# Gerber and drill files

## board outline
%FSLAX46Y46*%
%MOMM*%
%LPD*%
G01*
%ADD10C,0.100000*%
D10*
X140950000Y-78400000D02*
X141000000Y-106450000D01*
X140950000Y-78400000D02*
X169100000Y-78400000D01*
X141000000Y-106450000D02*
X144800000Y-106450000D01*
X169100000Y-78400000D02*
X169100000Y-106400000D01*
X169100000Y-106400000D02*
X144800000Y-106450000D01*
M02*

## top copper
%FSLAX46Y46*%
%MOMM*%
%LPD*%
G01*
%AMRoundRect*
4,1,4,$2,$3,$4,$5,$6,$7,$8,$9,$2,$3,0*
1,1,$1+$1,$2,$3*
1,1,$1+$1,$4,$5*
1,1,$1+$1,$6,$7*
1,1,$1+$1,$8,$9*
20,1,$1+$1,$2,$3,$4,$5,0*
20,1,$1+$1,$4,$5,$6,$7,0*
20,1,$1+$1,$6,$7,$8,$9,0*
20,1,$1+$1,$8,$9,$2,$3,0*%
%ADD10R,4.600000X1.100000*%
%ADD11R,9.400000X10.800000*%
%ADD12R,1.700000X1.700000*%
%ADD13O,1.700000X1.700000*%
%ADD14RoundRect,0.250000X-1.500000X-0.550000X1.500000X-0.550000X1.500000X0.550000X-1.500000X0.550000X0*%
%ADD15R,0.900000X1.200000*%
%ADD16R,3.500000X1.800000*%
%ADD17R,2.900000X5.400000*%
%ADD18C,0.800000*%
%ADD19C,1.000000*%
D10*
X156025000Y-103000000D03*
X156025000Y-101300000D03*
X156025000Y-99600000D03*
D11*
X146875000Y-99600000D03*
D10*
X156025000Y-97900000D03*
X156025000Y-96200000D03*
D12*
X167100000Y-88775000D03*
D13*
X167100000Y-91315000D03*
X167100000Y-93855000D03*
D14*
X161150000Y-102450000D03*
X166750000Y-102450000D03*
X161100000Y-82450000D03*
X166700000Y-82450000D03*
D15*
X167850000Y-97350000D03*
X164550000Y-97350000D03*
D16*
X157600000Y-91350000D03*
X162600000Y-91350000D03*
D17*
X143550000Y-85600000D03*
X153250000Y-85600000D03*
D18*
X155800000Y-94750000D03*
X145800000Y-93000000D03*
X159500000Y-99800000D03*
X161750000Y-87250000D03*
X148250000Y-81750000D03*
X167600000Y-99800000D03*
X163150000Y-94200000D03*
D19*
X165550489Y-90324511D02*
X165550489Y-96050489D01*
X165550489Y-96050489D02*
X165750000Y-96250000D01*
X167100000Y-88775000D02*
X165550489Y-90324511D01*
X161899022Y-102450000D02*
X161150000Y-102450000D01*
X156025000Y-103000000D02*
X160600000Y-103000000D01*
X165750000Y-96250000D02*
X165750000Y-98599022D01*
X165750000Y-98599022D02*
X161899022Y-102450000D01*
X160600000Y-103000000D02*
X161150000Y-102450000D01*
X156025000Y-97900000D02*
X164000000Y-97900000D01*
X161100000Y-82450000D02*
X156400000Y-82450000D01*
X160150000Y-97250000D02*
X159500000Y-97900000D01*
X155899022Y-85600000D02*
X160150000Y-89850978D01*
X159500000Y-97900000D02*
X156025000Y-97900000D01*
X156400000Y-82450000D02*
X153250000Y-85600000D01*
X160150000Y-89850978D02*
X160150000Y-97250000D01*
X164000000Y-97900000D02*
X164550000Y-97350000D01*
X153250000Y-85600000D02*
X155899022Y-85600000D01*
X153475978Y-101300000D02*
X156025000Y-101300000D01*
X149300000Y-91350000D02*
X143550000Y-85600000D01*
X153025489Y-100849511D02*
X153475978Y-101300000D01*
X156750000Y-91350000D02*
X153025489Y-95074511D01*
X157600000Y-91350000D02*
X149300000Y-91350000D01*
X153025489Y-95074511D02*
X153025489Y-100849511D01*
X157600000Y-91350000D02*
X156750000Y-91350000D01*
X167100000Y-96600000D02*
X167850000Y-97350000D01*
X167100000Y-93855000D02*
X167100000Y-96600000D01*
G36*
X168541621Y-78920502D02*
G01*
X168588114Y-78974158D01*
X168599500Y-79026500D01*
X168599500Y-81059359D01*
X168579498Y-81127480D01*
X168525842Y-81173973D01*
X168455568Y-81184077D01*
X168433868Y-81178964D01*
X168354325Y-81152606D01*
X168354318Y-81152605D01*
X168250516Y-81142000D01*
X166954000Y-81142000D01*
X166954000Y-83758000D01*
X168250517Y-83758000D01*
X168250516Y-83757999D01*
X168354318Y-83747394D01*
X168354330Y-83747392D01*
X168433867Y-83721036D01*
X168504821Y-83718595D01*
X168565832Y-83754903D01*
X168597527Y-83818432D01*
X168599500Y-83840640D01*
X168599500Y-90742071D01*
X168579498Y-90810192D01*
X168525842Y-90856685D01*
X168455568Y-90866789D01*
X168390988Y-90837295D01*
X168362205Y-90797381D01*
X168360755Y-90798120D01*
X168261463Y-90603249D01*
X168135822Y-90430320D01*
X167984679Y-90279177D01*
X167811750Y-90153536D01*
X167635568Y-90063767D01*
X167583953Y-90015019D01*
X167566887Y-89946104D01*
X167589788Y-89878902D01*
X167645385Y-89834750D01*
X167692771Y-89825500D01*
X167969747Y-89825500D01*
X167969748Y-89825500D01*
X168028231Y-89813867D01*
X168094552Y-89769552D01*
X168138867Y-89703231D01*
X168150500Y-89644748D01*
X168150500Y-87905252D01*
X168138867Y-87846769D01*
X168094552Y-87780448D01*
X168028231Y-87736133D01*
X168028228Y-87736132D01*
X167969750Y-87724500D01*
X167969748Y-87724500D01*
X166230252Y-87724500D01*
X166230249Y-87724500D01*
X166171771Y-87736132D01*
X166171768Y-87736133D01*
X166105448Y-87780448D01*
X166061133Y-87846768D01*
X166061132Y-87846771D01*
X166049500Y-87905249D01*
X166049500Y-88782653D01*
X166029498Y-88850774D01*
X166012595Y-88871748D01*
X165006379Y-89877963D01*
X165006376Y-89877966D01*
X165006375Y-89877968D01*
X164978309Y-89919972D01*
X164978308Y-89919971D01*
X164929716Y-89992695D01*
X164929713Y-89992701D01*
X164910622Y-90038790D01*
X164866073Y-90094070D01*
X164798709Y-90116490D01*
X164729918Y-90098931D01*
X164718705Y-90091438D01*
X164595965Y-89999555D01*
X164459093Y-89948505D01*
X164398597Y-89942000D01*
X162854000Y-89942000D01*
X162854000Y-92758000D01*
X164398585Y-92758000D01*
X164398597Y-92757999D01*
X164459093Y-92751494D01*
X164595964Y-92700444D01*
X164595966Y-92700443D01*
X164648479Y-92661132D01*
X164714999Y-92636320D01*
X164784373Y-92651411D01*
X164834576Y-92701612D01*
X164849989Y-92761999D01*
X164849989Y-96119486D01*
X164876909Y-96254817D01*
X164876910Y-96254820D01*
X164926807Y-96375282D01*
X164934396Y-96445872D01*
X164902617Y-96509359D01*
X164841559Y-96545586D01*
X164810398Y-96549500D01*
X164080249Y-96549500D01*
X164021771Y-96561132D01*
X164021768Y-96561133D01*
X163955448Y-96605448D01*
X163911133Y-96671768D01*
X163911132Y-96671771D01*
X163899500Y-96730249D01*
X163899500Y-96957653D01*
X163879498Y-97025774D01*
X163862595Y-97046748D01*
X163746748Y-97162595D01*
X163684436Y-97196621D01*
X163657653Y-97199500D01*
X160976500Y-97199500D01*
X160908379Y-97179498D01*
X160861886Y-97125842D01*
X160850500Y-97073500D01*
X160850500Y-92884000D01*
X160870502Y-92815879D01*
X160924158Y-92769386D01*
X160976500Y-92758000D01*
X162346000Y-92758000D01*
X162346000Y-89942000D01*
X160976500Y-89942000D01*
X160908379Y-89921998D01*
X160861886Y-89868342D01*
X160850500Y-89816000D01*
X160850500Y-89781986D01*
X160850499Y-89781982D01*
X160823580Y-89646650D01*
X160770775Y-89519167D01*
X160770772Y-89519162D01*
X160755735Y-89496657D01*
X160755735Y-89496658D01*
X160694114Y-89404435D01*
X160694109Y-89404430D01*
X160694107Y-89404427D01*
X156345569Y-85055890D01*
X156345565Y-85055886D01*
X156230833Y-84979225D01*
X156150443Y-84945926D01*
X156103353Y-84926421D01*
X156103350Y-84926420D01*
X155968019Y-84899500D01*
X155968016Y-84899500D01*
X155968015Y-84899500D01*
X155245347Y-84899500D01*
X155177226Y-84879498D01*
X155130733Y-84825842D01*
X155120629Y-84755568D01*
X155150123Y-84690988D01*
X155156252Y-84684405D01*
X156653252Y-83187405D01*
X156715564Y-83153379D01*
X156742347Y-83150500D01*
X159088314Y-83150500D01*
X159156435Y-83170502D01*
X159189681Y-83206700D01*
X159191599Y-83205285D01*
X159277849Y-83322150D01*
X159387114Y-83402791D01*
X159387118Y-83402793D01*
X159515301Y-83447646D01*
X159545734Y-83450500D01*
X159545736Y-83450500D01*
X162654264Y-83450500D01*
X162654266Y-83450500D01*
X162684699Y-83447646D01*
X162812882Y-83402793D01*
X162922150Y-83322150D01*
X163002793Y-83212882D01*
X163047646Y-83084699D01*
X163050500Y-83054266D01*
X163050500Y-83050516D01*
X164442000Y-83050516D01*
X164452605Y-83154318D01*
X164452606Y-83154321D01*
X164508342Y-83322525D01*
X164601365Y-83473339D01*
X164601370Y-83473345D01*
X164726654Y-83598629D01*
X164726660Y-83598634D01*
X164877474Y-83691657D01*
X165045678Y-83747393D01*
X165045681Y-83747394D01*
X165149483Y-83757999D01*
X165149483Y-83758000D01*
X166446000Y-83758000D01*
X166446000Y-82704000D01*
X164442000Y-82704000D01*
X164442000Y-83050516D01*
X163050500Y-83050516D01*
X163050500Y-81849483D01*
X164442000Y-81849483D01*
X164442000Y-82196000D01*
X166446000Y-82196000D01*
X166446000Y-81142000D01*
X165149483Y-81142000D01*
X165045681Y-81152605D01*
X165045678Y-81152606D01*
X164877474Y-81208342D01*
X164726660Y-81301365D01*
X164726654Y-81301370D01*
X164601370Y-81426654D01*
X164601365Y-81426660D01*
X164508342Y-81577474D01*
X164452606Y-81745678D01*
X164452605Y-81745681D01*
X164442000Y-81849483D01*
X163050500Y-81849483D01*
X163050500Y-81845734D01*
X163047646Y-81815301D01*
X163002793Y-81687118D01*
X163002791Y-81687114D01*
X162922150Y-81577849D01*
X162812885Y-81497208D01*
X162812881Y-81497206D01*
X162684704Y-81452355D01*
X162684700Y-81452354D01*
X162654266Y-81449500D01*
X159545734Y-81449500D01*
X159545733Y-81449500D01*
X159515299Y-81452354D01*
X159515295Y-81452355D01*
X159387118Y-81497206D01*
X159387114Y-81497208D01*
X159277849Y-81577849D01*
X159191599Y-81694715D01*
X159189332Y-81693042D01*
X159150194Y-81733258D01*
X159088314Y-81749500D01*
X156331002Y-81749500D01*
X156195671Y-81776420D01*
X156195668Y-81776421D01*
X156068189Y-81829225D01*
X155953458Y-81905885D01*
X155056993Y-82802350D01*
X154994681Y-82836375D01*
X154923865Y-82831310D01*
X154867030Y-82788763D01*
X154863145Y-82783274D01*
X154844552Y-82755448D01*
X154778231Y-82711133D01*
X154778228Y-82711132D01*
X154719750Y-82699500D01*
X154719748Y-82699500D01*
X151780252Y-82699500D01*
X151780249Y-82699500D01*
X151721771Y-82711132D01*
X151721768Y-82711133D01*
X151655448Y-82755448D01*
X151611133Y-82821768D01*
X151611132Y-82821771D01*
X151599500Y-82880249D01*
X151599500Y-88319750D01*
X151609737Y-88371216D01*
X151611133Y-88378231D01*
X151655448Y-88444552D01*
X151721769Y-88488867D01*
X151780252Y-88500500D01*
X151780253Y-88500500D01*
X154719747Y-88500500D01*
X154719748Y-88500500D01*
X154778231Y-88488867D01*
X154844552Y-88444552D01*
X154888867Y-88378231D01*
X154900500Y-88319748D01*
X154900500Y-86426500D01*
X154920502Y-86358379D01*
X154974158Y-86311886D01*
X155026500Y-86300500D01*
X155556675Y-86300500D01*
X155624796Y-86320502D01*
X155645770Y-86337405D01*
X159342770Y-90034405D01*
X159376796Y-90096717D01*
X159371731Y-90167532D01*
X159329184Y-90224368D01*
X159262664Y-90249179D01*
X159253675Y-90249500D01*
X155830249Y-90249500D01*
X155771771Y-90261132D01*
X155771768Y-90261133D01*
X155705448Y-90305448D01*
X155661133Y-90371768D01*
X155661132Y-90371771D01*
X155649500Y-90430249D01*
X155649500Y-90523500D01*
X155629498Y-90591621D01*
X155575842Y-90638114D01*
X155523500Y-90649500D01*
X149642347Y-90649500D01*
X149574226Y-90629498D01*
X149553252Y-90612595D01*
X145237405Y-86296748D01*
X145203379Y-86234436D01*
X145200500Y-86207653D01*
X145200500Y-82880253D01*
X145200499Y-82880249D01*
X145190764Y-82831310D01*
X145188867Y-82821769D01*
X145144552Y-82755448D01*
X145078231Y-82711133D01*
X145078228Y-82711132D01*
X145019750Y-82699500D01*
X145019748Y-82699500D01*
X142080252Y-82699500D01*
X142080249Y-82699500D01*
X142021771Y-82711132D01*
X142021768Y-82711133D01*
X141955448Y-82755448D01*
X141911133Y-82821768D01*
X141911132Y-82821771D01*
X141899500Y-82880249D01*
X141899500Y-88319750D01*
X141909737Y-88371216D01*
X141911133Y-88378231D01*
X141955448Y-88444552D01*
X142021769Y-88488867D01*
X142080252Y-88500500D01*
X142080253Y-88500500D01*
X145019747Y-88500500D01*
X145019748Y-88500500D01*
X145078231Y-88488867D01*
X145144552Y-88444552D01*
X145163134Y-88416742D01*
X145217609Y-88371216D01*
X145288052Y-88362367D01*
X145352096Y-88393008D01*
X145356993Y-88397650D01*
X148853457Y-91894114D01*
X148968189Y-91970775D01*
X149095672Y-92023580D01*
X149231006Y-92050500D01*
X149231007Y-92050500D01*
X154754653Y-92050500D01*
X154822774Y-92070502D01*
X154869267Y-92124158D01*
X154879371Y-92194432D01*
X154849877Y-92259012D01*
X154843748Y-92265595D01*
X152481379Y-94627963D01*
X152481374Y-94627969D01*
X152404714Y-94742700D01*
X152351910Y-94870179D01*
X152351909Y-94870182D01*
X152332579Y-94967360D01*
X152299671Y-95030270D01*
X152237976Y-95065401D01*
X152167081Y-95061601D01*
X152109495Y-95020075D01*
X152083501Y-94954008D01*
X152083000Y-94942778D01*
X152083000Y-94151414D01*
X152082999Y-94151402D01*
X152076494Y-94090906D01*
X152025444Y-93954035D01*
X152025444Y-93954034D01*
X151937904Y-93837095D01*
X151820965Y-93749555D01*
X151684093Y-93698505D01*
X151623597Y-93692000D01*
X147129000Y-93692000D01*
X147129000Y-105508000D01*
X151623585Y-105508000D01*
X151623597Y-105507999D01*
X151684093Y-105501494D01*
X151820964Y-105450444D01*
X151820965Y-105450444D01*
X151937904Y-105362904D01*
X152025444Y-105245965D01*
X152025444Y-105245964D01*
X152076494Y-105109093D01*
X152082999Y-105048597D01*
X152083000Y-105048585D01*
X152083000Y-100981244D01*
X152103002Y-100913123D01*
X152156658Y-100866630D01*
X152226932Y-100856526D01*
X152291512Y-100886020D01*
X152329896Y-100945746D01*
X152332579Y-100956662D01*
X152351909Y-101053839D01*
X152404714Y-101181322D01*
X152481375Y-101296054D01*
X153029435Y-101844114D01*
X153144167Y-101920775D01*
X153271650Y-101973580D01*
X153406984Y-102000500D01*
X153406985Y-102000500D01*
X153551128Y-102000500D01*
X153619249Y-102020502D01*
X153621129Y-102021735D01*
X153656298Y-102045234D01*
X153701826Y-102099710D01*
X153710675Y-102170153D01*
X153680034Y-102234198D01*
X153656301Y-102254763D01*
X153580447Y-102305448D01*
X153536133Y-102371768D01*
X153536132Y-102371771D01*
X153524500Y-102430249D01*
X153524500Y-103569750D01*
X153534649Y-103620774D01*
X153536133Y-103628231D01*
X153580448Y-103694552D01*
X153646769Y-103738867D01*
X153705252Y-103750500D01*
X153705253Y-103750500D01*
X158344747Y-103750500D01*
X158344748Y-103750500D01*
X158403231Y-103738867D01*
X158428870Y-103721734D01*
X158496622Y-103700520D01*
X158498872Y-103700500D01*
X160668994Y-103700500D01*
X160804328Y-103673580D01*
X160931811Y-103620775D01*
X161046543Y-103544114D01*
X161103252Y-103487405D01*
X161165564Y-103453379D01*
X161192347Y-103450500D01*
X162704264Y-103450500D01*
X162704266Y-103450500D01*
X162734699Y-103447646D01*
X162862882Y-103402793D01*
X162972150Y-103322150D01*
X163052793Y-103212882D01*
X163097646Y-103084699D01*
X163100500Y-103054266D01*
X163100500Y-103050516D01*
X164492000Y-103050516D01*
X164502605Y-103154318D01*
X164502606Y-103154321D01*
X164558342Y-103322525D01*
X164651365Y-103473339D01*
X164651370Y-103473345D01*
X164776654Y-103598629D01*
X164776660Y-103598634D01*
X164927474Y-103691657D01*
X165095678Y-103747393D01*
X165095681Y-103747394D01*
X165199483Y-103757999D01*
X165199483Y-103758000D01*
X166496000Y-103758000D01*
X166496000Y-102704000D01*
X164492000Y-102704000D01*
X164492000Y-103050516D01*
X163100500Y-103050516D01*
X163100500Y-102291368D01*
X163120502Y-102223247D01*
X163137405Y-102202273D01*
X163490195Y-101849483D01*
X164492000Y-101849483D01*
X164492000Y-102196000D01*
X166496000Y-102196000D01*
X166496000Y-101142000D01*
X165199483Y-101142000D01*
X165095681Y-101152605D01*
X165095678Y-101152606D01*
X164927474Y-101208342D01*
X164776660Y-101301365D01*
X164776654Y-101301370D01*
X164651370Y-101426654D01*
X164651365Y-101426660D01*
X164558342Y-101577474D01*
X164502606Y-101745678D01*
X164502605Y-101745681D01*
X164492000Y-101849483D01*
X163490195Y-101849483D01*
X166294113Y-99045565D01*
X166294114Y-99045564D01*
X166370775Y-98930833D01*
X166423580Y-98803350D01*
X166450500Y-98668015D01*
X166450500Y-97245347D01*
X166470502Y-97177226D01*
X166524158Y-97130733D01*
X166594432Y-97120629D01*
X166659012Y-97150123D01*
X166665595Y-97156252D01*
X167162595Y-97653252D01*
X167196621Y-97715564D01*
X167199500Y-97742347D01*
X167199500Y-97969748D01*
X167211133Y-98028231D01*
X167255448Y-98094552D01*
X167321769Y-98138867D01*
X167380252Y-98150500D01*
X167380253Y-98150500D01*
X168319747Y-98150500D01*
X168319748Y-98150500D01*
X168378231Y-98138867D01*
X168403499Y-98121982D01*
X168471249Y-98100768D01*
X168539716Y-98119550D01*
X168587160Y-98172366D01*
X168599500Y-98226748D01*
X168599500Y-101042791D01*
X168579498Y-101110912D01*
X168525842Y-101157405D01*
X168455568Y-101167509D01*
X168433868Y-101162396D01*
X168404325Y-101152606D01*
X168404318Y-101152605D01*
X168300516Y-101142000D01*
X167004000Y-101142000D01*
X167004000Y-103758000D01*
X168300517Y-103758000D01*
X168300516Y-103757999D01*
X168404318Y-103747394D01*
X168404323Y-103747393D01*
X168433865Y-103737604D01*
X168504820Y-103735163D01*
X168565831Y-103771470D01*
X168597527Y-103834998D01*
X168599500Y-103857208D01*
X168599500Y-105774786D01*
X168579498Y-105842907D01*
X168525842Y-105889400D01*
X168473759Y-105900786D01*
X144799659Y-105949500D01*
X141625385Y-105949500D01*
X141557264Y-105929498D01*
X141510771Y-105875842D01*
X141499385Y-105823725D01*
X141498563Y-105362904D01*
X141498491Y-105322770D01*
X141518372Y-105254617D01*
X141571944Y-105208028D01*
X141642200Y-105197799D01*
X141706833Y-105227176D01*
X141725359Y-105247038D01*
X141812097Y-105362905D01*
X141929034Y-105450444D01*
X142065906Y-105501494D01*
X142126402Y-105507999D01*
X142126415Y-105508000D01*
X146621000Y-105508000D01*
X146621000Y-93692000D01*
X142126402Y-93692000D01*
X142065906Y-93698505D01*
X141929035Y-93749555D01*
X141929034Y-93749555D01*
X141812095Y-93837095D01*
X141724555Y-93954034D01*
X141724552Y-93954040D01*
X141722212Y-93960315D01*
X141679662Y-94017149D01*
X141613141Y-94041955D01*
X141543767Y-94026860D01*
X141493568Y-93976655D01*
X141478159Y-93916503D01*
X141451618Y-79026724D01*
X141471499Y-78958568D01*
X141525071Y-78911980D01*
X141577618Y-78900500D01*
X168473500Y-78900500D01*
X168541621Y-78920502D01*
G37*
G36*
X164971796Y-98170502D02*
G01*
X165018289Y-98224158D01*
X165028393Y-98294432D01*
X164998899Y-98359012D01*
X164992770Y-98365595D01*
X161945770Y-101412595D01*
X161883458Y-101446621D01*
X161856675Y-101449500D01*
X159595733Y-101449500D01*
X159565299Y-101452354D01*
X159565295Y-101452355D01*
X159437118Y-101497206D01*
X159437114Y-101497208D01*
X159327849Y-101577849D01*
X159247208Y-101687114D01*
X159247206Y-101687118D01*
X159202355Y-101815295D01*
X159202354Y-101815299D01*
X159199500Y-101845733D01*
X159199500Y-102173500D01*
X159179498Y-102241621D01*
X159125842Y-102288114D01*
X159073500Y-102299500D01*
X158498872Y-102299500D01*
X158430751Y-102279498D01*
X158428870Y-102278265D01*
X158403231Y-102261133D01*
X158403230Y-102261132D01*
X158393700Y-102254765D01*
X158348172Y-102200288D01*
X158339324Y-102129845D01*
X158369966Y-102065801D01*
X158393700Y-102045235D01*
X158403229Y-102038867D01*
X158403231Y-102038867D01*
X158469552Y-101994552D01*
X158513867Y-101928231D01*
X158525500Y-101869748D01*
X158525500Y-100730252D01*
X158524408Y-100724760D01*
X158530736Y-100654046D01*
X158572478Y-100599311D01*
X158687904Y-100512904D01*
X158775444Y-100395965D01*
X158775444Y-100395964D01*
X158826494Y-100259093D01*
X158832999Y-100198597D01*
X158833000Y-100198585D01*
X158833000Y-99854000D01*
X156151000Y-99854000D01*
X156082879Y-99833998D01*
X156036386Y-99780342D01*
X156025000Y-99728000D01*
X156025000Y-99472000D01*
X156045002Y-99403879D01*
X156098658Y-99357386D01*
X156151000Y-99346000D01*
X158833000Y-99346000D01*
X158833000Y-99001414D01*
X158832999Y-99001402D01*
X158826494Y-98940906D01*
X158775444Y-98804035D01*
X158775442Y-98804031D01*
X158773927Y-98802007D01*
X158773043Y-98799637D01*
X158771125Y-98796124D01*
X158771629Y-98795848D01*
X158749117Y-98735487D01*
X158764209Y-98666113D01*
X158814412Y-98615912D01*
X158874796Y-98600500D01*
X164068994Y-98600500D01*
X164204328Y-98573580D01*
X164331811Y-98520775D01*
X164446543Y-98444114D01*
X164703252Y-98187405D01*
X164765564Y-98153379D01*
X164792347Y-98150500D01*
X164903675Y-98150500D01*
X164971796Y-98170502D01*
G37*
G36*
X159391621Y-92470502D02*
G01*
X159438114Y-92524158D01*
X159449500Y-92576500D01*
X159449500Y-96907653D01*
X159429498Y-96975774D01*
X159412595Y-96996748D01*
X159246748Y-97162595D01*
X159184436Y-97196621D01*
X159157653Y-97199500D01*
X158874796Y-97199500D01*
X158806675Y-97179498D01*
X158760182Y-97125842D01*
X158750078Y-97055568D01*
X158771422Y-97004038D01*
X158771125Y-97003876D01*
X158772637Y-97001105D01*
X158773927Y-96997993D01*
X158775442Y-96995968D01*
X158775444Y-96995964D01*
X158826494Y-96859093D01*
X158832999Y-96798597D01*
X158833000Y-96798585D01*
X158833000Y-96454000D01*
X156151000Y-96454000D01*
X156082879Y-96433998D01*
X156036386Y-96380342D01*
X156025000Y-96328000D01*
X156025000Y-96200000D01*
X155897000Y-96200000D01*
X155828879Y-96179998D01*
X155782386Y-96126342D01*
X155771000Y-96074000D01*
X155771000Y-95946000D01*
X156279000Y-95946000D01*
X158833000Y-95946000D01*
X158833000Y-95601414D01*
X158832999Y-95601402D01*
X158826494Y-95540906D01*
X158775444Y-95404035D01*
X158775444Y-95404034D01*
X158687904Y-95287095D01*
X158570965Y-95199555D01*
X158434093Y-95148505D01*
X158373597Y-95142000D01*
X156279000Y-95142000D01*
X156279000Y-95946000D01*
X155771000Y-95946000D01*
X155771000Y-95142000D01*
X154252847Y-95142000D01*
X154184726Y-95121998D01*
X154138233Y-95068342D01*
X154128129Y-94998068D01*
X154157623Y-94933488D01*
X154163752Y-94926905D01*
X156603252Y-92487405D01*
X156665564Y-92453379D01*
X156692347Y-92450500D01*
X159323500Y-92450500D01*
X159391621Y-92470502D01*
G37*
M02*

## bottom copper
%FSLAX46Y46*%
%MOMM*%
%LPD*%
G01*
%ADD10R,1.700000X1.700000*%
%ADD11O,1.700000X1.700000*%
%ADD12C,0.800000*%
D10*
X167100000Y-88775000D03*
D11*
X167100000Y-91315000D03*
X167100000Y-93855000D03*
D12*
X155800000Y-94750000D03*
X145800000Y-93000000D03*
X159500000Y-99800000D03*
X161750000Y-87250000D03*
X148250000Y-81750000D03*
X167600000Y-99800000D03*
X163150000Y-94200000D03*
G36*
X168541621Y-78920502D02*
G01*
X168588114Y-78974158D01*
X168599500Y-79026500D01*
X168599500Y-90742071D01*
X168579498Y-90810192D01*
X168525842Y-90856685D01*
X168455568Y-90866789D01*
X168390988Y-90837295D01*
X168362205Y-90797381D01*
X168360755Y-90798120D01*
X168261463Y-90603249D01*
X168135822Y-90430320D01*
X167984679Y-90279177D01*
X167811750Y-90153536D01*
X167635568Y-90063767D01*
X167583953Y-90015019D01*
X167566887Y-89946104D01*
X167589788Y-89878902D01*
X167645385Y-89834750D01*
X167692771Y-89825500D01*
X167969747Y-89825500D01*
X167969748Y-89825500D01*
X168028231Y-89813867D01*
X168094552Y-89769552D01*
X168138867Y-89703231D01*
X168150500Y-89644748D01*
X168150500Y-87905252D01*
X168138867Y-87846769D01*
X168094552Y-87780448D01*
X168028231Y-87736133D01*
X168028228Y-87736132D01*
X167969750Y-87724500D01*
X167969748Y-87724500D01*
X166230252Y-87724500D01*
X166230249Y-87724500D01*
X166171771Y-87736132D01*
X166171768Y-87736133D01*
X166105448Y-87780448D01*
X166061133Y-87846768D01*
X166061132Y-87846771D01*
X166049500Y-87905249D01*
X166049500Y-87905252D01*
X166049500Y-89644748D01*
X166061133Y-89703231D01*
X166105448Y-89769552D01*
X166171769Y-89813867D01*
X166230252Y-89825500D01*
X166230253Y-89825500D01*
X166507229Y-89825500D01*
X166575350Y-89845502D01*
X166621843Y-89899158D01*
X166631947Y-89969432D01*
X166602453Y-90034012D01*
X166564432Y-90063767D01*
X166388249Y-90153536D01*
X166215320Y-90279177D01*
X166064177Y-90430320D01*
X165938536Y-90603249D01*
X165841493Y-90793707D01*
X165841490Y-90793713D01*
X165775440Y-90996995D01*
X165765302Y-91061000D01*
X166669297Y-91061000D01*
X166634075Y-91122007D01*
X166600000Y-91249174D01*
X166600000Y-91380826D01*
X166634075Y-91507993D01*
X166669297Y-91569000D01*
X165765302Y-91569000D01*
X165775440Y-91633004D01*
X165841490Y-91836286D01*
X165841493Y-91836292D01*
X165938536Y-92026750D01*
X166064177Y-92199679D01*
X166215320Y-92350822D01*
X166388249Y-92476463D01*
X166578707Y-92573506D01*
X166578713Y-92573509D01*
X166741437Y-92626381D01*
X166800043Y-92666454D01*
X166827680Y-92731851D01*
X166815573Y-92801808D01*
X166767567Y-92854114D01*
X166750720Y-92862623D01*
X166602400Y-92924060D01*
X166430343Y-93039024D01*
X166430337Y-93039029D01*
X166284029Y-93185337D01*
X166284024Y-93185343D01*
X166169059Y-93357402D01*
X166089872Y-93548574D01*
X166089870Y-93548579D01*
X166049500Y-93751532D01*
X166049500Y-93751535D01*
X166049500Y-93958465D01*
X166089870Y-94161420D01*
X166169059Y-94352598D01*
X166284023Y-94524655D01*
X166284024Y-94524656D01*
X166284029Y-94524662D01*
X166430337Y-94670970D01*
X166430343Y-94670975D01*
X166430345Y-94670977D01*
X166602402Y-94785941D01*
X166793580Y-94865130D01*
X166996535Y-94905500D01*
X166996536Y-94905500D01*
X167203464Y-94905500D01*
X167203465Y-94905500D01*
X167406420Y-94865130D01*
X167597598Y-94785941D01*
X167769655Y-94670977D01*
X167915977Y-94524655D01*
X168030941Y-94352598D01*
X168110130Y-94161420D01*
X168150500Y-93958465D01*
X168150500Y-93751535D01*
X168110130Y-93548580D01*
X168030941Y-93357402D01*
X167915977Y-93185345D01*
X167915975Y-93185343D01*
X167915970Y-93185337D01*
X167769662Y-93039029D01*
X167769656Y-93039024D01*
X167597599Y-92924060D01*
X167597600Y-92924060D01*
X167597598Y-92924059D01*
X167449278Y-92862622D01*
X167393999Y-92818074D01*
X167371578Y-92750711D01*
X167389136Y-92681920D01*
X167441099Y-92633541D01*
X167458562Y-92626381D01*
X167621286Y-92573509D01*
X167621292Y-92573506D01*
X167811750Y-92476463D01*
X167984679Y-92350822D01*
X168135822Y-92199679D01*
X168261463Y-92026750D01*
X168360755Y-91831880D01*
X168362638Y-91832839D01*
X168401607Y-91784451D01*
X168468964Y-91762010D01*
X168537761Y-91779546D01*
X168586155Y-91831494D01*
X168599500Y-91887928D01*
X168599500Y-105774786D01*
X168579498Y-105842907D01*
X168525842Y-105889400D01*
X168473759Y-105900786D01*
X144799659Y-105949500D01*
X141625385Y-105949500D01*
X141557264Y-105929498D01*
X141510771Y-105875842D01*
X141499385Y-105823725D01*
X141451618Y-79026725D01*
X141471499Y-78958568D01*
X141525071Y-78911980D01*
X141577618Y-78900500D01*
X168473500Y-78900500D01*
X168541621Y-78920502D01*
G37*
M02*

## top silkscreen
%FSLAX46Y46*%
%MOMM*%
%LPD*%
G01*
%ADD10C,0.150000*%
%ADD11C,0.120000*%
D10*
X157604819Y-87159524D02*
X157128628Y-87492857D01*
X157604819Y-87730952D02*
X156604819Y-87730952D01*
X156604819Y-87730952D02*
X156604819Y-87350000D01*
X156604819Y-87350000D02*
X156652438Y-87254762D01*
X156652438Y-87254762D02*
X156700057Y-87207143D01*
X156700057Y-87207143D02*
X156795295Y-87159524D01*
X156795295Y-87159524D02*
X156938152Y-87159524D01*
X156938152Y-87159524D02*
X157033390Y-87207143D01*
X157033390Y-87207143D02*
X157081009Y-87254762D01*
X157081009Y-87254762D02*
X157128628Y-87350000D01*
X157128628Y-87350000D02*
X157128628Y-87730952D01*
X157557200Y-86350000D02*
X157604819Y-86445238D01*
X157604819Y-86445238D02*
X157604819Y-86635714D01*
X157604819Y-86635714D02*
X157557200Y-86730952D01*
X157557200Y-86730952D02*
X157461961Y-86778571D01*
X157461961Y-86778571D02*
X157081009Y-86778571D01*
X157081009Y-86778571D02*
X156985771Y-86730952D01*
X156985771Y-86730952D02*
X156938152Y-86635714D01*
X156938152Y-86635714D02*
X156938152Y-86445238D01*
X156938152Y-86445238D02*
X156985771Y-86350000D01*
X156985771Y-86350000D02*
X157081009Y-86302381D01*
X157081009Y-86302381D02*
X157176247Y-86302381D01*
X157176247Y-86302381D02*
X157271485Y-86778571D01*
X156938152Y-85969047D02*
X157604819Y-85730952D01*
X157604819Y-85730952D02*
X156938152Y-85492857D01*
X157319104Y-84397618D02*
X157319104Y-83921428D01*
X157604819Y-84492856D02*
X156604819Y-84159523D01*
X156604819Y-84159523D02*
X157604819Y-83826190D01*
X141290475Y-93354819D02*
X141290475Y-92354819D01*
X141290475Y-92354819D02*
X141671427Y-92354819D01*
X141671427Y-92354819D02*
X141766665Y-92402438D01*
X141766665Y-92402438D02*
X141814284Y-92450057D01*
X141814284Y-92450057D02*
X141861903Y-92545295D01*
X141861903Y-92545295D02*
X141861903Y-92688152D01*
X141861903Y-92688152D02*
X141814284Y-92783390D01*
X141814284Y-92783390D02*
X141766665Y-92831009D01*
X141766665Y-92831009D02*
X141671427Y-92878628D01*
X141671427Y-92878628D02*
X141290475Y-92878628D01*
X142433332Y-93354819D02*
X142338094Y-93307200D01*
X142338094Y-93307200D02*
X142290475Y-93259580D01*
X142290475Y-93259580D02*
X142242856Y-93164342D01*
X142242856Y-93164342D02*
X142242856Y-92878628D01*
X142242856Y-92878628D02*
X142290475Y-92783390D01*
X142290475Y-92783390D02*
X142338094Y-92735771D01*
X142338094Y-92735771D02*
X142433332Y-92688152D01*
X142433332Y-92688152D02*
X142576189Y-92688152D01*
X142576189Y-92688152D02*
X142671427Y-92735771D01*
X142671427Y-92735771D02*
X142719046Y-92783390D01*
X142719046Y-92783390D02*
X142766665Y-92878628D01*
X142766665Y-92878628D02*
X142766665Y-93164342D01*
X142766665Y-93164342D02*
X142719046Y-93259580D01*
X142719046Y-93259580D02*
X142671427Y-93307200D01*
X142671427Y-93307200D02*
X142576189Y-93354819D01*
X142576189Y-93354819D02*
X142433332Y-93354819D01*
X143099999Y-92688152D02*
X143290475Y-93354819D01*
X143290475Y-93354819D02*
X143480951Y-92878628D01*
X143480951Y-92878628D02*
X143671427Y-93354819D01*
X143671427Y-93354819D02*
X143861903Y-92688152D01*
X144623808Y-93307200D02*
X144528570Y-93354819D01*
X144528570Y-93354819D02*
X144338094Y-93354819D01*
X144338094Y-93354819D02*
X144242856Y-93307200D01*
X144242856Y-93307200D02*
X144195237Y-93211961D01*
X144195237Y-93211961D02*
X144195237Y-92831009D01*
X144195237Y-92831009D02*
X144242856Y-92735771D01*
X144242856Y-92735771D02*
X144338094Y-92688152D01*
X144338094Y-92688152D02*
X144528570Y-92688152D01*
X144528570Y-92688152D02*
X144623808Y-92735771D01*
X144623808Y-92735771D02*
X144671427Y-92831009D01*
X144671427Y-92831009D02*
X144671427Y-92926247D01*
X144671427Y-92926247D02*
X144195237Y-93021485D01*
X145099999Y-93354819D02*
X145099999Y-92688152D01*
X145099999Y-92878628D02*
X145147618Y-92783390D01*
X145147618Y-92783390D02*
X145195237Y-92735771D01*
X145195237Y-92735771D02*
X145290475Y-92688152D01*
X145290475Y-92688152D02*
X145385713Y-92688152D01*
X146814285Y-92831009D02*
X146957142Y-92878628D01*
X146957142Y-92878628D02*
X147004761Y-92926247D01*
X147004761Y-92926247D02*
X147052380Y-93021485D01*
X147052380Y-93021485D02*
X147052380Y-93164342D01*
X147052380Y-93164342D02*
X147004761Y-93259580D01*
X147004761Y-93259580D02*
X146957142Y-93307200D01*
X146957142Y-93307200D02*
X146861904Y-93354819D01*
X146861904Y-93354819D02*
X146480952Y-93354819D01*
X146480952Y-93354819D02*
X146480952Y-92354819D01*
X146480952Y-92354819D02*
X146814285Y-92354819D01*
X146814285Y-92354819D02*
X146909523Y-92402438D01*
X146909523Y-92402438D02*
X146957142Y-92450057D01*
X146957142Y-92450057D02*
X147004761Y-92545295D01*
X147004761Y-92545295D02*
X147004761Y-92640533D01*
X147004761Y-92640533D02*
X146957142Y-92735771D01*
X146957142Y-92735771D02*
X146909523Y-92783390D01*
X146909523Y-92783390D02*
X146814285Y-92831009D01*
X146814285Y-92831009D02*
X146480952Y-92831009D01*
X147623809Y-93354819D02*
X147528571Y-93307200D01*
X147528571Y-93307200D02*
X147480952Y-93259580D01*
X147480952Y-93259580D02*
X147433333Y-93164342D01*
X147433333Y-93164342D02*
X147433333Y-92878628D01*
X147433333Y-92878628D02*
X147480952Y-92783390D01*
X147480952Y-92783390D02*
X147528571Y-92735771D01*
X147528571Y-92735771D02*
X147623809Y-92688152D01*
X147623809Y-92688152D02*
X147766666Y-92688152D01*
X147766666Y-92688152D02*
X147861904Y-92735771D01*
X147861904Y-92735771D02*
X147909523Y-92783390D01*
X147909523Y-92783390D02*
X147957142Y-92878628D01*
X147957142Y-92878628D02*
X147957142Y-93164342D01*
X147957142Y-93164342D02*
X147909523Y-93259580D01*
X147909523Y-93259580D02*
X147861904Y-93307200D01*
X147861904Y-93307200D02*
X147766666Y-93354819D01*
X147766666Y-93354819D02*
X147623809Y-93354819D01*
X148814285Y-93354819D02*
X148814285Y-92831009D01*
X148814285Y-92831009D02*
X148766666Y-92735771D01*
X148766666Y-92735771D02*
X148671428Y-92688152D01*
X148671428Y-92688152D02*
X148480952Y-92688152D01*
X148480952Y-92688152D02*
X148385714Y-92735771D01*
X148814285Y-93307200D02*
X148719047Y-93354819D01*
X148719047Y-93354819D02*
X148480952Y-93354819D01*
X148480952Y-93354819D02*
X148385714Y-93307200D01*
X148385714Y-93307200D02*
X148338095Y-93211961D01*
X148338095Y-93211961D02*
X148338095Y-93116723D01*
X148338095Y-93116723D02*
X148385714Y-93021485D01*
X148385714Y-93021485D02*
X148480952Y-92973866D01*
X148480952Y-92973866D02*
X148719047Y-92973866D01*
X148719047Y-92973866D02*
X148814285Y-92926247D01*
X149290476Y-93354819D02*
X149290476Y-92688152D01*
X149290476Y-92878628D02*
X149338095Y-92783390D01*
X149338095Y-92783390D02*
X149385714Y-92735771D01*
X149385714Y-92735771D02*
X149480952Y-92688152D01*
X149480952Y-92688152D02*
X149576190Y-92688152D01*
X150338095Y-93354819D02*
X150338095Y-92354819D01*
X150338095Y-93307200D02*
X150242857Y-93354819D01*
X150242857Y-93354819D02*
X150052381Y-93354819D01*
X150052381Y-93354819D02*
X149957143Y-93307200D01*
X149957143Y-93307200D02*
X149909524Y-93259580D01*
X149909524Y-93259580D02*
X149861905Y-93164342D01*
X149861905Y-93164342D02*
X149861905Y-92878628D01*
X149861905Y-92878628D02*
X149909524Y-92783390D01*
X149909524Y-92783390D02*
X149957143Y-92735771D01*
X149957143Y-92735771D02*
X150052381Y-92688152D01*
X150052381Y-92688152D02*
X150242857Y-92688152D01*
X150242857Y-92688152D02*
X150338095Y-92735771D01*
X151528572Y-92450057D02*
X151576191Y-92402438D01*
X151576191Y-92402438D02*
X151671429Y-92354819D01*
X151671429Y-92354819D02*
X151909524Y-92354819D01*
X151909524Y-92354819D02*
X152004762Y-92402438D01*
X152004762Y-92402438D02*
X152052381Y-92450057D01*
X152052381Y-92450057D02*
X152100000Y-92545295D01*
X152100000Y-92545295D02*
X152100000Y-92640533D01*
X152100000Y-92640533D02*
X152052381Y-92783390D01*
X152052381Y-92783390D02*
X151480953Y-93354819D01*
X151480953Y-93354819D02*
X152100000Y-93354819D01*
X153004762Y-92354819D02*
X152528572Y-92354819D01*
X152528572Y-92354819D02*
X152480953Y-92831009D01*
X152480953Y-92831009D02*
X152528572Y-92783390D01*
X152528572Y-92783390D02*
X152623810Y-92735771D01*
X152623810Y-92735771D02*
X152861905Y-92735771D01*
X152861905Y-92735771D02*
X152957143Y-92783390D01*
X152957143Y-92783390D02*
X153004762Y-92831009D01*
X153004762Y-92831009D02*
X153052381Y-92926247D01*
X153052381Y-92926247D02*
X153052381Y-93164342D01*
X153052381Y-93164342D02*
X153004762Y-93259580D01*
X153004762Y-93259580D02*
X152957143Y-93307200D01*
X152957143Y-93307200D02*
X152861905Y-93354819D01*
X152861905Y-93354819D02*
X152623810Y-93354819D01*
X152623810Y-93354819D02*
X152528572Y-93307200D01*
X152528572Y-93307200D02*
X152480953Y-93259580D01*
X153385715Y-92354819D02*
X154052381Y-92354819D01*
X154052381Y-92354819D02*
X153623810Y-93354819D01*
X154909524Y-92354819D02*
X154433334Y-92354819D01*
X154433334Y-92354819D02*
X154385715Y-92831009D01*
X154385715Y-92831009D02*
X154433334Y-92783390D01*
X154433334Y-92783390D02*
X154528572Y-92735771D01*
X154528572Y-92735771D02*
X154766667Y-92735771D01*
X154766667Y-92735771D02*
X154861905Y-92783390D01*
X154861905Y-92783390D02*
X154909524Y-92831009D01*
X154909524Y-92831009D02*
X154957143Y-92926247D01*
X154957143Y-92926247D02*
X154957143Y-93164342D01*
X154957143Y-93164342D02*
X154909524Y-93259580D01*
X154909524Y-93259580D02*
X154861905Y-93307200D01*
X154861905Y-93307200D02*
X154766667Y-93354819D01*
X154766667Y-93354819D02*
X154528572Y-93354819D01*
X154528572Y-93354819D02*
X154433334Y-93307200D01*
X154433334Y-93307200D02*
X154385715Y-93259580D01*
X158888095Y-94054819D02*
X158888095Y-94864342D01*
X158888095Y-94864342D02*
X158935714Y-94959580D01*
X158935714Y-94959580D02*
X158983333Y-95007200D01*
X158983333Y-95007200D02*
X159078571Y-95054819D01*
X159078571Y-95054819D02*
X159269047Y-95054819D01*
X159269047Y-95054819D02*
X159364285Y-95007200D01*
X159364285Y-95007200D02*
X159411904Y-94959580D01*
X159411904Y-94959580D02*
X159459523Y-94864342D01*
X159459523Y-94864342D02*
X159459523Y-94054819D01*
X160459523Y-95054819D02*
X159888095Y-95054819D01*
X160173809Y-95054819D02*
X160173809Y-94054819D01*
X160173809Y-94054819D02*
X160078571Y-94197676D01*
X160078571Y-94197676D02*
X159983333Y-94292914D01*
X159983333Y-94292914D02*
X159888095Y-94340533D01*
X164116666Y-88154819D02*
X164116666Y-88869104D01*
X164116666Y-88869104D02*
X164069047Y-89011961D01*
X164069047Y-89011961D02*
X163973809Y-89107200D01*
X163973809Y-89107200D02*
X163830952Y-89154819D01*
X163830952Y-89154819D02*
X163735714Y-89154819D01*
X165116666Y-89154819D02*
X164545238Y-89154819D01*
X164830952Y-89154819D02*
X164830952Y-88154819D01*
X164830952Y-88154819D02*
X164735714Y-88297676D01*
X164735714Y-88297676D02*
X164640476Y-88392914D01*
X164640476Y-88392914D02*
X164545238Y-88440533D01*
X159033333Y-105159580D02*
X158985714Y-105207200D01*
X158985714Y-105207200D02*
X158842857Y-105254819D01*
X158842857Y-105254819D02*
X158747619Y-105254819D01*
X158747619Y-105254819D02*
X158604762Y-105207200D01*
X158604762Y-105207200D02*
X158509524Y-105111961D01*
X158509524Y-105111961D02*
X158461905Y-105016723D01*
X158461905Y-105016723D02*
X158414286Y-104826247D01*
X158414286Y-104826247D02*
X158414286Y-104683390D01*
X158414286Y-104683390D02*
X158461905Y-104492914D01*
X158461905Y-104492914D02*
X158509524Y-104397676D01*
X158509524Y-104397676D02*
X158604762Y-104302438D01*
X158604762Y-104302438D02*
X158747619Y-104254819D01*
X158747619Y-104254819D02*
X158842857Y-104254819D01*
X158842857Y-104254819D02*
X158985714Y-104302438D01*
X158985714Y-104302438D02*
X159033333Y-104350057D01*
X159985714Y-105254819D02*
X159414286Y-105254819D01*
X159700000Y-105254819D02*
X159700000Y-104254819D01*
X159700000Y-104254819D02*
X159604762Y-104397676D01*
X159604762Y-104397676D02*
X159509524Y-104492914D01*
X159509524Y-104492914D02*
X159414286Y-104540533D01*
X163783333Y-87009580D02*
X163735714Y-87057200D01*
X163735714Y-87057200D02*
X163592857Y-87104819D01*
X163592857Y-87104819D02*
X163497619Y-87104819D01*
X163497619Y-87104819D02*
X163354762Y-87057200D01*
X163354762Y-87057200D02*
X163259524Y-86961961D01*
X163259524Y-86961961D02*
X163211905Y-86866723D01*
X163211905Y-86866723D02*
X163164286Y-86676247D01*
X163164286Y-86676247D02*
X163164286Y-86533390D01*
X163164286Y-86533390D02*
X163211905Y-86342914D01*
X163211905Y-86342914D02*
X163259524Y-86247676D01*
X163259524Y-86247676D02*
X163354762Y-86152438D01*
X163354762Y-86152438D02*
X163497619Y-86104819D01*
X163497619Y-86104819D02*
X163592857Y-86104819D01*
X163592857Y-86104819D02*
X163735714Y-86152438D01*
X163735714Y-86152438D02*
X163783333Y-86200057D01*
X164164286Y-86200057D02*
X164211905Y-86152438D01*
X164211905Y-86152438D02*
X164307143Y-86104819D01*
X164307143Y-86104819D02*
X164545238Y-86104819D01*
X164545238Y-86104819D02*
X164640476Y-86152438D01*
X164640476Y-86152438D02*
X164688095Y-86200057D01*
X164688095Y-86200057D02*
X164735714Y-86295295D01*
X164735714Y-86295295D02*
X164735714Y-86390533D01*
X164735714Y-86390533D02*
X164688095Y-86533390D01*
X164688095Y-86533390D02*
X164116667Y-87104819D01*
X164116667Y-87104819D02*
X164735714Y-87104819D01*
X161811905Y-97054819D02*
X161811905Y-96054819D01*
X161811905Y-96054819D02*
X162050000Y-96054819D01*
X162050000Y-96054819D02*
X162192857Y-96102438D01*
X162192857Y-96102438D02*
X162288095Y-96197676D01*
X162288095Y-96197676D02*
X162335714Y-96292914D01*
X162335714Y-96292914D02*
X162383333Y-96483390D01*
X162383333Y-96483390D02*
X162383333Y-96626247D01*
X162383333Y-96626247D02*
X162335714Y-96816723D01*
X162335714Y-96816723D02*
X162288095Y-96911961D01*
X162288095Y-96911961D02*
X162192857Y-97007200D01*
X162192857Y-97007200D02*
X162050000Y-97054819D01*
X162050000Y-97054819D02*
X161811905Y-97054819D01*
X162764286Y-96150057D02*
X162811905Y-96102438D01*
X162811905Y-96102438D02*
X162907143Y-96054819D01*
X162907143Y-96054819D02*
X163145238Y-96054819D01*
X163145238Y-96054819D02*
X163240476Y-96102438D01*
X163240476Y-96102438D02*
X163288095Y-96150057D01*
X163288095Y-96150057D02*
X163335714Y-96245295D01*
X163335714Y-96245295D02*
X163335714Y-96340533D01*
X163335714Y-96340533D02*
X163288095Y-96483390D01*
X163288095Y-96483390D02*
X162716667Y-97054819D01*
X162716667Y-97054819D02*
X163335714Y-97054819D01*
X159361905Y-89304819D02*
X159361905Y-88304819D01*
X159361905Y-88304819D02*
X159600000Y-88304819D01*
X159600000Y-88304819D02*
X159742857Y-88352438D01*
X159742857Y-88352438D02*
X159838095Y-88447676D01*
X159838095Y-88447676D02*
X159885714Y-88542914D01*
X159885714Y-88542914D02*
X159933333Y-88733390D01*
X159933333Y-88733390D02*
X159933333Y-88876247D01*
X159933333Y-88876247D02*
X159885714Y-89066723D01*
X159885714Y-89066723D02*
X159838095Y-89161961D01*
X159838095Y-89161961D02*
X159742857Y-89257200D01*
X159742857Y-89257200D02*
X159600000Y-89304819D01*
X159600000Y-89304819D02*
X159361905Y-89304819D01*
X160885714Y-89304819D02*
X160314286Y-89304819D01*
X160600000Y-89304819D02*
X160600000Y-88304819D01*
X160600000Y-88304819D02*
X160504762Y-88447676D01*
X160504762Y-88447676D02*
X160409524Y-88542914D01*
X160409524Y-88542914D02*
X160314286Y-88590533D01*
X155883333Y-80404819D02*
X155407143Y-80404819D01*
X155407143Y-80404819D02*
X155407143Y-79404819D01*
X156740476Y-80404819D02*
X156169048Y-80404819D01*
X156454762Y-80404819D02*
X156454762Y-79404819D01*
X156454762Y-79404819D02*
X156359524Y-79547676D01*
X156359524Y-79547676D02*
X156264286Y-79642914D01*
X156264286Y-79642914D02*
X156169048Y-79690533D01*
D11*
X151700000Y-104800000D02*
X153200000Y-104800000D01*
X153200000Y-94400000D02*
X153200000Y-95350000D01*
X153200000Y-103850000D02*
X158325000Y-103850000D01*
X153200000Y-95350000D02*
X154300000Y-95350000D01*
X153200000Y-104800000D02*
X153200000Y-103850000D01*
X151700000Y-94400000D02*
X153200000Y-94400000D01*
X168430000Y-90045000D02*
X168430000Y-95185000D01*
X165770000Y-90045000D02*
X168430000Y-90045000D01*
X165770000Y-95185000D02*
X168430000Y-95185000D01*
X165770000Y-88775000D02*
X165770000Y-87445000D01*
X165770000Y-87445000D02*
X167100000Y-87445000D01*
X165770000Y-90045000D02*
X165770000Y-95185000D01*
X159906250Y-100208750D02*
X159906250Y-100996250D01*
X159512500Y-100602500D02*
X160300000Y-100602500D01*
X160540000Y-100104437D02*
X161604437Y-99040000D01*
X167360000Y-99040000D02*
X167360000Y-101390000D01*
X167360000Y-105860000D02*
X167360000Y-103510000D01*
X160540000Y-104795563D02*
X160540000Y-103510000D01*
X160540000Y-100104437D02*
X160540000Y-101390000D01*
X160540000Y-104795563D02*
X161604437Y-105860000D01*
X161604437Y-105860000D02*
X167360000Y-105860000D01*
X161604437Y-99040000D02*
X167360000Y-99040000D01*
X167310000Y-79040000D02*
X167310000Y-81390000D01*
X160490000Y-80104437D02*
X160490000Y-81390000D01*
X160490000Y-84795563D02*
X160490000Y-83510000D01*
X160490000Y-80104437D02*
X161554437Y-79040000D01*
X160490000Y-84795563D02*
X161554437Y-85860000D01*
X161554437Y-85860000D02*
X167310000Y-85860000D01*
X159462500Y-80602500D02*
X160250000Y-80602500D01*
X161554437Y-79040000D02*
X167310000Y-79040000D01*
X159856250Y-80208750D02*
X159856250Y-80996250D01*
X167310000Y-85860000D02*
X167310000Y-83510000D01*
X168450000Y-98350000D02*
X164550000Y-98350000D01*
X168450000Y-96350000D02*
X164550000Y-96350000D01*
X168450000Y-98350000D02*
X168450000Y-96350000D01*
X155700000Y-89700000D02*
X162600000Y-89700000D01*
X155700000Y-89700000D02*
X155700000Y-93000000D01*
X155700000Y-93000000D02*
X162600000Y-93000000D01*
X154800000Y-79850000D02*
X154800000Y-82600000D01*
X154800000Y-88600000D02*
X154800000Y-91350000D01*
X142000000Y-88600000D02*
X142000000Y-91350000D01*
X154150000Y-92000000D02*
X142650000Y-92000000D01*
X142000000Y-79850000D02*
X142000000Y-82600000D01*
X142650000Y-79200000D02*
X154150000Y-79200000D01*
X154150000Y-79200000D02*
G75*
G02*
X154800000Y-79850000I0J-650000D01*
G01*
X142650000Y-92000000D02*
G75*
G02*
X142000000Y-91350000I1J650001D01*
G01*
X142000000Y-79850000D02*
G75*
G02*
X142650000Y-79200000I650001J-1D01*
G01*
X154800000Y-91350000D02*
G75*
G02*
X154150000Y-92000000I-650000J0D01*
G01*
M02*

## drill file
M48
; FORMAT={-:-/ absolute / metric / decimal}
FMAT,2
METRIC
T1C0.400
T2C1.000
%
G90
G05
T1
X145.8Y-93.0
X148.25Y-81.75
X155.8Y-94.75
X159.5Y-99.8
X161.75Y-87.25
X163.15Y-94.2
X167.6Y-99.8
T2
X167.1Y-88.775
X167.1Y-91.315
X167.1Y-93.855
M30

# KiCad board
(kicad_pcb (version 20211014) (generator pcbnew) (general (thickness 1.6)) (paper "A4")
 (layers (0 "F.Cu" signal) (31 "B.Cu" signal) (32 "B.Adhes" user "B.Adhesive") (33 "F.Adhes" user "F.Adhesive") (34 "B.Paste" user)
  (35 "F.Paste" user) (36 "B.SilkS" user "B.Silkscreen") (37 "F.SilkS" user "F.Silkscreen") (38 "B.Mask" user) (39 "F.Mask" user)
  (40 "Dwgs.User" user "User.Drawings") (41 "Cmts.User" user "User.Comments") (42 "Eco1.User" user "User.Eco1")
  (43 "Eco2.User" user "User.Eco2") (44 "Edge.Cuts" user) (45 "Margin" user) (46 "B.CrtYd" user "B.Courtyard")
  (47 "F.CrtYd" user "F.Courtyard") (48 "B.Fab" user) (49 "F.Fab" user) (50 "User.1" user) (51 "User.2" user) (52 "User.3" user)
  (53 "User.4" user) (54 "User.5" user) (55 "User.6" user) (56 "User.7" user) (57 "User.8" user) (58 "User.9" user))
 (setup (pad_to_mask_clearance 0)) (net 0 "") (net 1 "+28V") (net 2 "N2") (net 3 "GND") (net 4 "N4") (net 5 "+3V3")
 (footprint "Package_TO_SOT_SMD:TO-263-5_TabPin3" (layer "F.Cu") (at 150.25 99.6 180)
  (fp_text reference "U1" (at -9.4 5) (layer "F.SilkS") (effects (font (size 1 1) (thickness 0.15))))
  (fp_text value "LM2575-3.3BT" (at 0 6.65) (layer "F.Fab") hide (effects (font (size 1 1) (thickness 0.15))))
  (fp_line (start -1.45 -5.2) (end -2.95 -5.2) (layer "F.SilkS") (width 0.12))
  (fp_line (start -2.95 5.2) (end -2.95 4.25) (layer "F.SilkS") (width 0.12))
  (fp_line (start -2.95 -4.25) (end -8.075 -4.25) (layer "F.SilkS") (width 0.12))
  (fp_line (start -2.95 4.25) (end -4.05 4.25) (layer "F.SilkS") (width 0.12))
  (fp_line (start -2.95 -5.2) (end -2.95 -4.25) (layer "F.SilkS") (width 0.12))
  (fp_line (start -1.45 5.2) (end -2.95 5.2) (layer "F.SilkS") (width 0.12))
  (pad "" smd rect (at 0.95 -2.775 180) (size 4.55 5.25) (layers "F.Paste"))
  (pad "" smd rect (at 5.8 -2.775 180) (size 4.55 5.25) (layers "F.Paste"))
  (pad "" smd rect (at 5.8 2.775 180) (size 4.55 5.25) (layers "F.Paste"))
  (pad "" smd rect (at 0.95 2.775 180) (size 4.55 5.25) (layers "F.Paste"))
  (pad "1" smd rect (at -5.775 -3.4 180) (size 4.6 1.1) (layers "F.Cu" "F.Paste" "F.Mask") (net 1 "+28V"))
  (pad "2" smd rect (at -5.775 -1.7 180) (size 4.6 1.1) (layers "F.Cu" "F.Paste" "F.Mask") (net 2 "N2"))
  (pad "3" smd rect (at -5.775 0 180) (size 4.6 1.1) (layers "F.Cu" "F.Paste" "F.Mask") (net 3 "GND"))
  (pad "3" smd rect (at 3.375 0 180) (size 9.4 10.8) (layers "F.Cu" "F.Mask") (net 3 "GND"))
  (pad "4" smd rect (at -5.775 1.7 180) (size 4.6 1.1) (layers "F.Cu" "F.Paste" "F.Mask") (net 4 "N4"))
  (pad "5" smd rect (at -5.775 3.4 180) (size 4.6 1.1) (layers "F.Cu" "F.Paste" "F.Mask") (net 3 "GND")))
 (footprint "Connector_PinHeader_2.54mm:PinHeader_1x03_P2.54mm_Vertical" (layer "F.Cu") (at 167.1 88.775)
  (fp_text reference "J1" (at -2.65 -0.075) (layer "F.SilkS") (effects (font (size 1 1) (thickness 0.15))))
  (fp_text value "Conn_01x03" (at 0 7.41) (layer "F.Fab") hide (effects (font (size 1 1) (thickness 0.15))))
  (fp_line (start 1.33 1.27) (end 1.33 6.41) (layer "F.SilkS") (width 0.12))
  (fp_line (start -1.33 1.27) (end 1.33 1.27) (layer "F.SilkS") (width 0.12))
  (fp_line (start -1.33 6.41) (end 1.33 6.41) (layer "F.SilkS") (width 0.12))
  (fp_line (start -1.33 0) (end -1.33 -1.33) (layer "F.SilkS") (width 0.12))
  (fp_line (start -1.33 -1.33) (end 0 -1.33) (layer "F.SilkS") (width 0.12))
  (fp_line (start -1.33 1.27) (end -1.33 6.41) (layer "F.SilkS") (width 0.12))
  (pad "1" thru_hole rect (at 0 0) (size 1.7 1.7) (drill 1) (layers *.Cu *.Mask) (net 1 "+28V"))
  (pad "2" thru_hole oval (at 0 2.54) (size 1.7 1.7) (drill 1) (layers *.Cu *.Mask) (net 3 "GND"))
  (pad "3" thru_hole oval (at 0 5.08) (size 1.7 1.7) (drill 1) (layers *.Cu *.Mask) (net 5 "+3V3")))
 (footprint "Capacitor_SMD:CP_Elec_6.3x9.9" (layer "F.Cu") (at 163.95 102.45)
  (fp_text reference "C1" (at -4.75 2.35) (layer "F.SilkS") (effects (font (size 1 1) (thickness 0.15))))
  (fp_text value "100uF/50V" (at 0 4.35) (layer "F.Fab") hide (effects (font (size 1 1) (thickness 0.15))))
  (fp_line (start -4.04375 -2.24125) (end -4.04375 -1.45375) (layer "F.SilkS") (width 0.12))
  (fp_line (start -4.4375 -1.8475) (end -3.65 -1.8475) (layer "F.SilkS") (width 0.12))
  (fp_line (start -3.41 -2.345563) (end -2.345563 -3.41) (layer "F.SilkS") (width 0.12))
  (fp_line (start 3.41 -3.41) (end 3.41 -1.06) (layer "F.SilkS") (width 0.12))
  (fp_line (start 3.41 3.41) (end 3.41 1.06) (layer "F.SilkS") (width 0.12))
  (fp_line (start -3.41 2.345563) (end -3.41 1.06) (layer "F.SilkS") (width 0.12))
  (fp_line (start -3.41 -2.345563) (end -3.41 -1.06) (layer "F.SilkS") (width 0.12))
  (fp_line (start -3.41 2.345563) (end -2.345563 3.41) (layer "F.SilkS") (width 0.12))
  (fp_line (start -2.345563 3.41) (end 3.41 3.41) (layer "F.SilkS") (width 0.12))
  (fp_line (start -2.345563 -3.41) (end 3.41 -3.41) (layer "F.SilkS") (width 0.12))
  (pad "1" smd roundrect (at -2.8 0) (size 3.5 1.6) (layers "F.Cu" "F.Paste" "F.Mask") (roundrect_rratio 0.15625) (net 1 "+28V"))
  (pad "2" smd roundrect (at 2.8 0) (size 3.5 1.6) (layers "F.Cu" "F.Paste" "F.Mask") (roundrect_rratio 0.15625) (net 3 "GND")))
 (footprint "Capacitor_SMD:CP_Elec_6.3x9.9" (layer "F.Cu") (at 163.9 82.45)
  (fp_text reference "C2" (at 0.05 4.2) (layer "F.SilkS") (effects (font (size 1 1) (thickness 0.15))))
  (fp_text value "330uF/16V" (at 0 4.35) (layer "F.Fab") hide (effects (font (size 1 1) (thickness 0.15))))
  (fp_line (start 3.41 -3.41) (end 3.41 -1.06) (layer "F.SilkS") (width 0.12))
  (fp_line (start -3.41 -2.345563) (end -3.41 -1.06) (layer "F.SilkS") (width 0.12))
  (fp_line (start -3.41 2.345563) (end -3.41 1.06) (layer "F.SilkS") (width 0.12))
  (fp_line (start -3.41 -2.345563) (end -2.345563 -3.41) (layer "F.SilkS") (width 0.12))
  (fp_line (start -3.41 2.345563) (end -2.345563 3.41) (layer "F.SilkS") (width 0.12))
  (fp_line (start -2.345563 3.41) (end 3.41 3.41) (layer "F.SilkS") (width 0.12))
  (fp_line (start -4.4375 -1.8475) (end -3.65 -1.8475) (layer "F.SilkS") (width 0.12))
  (fp_line (start -2.345563 -3.41) (end 3.41 -3.41) (layer "F.SilkS") (width 0.12))
  (fp_line (start -4.04375 -2.24125) (end -4.04375 -1.45375) (layer "F.SilkS") (width 0.12))
  (fp_line (start 3.41 3.41) (end 3.41 1.06) (layer "F.SilkS") (width 0.12))
  (pad "1" smd roundrect (at -2.8 0) (size 3.5 1.6) (layers "F.Cu" "F.Paste" "F.Mask") (roundrect_rratio 0.15625) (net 4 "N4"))
  (pad "2" smd roundrect (at 2.8 0) (size 3.5 1.6) (layers "F.Cu" "F.Paste" "F.Mask") (roundrect_rratio 0.15625) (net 3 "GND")))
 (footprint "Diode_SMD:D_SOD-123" (layer "F.Cu") (at 166.2 97.35 180)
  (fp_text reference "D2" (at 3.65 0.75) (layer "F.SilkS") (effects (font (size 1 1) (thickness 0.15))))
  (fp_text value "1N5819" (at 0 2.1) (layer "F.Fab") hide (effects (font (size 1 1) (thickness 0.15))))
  (fp_line (start -2.25 -1) (end 1.65 -1) (layer "F.SilkS") (width 0.12))
  (fp_line (start -2.25 1) (end 1.65 1) (layer "F.SilkS") (width 0.12))
  (fp_line (start -2.25 -1) (end -2.25 1) (layer "F.SilkS") (width 0.12))
  (pad "1" smd rect (at -1.65 0 180) (size 0.9 1.2) (layers "F.Cu" "F.Paste" "F.Mask") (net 5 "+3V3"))
  (pad "2" smd rect (at 1.65 0 180) (size 0.9 1.2) (layers "F.Cu" "F.Paste" "F.Mask") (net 4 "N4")))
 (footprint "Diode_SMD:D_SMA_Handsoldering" (layer "F.Cu") (at 160.1 91.35)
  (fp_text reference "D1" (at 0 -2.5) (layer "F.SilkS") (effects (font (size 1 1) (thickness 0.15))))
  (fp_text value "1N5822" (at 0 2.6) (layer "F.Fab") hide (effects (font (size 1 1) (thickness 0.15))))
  (fp_line (start -4.4 -1.65) (end 2.5 -1.65) (layer "F.SilkS") (width 0.12))
  (fp_line (start -4.4 -1.65) (end -4.4 1.65) (layer "F.SilkS") (width 0.12))
  (fp_line (start -4.4 1.65) (end 2.5 1.65) (layer "F.SilkS") (width 0.12))
  (pad "1" smd rect (at -2.5 0) (size 3.5 1.8) (layers "F.Cu" "F.Paste" "F.Mask") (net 2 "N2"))
  (pad "2" smd rect (at 2.5 0) (size 3.5 1.8) (layers "F.Cu" "F.Paste" "F.Mask") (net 3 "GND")))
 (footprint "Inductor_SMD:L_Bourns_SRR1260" (layer "F.Cu") (at 148.4 85.6)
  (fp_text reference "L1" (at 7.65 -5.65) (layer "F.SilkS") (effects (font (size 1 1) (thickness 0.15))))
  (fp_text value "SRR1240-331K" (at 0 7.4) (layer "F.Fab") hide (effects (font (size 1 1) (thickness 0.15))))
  (fp_line (start 6.4 -5.75) (end 6.4 -3) (layer "F.SilkS") (width 0.12))
  (fp_line (start 6.4 3) (end 6.4 5.75) (layer "F.SilkS") (width 0.12))
  (fp_line (start -6.4 3) (end -6.4 5.75) (layer "F.SilkS") (width 0.12))
  (fp_line (start 5.75 6.4) (end -5.75 6.4) (layer "F.SilkS") (width 0.12))
  (fp_line (start -6.4 -5.75) (end -6.4 -3) (layer "F.SilkS") (width 0.12))
  (fp_line (start -5.75 -6.4) (end 5.75 -6.4) (layer "F.SilkS") (width 0.12))
  (fp_arc (start 5.75 -6.4) (mid 6.209619 -6.209619) (end 6.4 -5.75) (layer "F.SilkS") (width 0.12))
  (fp_arc (start -5.75 6.4) (mid -6.209619 6.209619) (end -6.4 5.75) (layer "F.SilkS") (width 0.12))
  (fp_arc (start -6.4 -5.75) (mid -6.209619 -6.209619) (end -5.75 -6.4) (layer "F.SilkS") (width 0.12))
  (fp_arc (start 6.4 5.75) (mid 6.209619 6.209619) (end 5.75 6.4) (layer "F.SilkS") (width 0.12))
  (pad "1" smd rect (at -4.85 0) (size 2.9 5.4) (layers "F.Cu" "F.Paste" "F.Mask") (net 2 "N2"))
  (pad "2" smd rect (at 4.85 0) (size 2.9 5.4) (layers "F.Cu" "F.Paste" "F.Mask") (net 4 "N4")))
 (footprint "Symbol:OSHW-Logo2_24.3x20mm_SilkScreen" (layer "B.Cu") (at 154.7 92.05 180)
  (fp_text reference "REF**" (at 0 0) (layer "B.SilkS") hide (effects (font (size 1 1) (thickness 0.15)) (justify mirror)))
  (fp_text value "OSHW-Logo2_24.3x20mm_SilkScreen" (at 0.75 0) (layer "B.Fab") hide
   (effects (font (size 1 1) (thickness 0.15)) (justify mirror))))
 (gr_line (start 140.95 78.4) (end 141 106.45) (layer "Edge.Cuts") (width 0.1))
 (gr_line (start 140.95 78.4) (end 169.1 78.4) (layer "Edge.Cuts") (width 0.1))
 (gr_line (start 141 106.45) (end 144.8 106.45) (layer "Edge.Cuts") (width 0.1))
 (gr_line (start 169.1 78.4) (end 169.1 106.4) (layer "Edge.Cuts") (width 0.1))
 (gr_line (start 169.1 106.4) (end 144.8 106.45) (layer "Edge.Cuts") (width 0.1))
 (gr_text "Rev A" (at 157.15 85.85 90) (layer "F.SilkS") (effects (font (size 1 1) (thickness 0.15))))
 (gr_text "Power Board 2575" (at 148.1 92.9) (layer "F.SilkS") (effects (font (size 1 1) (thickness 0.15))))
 (segment (start 165.550489 90.324511) (end 165.550489 96.050489) (width 1) (layer "F.Cu") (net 1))
 (segment (start 165.550489 96.050489) (end 165.75 96.25) (width 1) (layer "F.Cu") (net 1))
 (segment (start 167.1 88.775) (end 165.550489 90.324511) (width 1) (layer "F.Cu") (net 1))
 (segment (start 161.899022 102.45) (end 161.15 102.45) (width 1) (layer "F.Cu") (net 1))
 (segment (start 156.025 103) (end 160.6 103) (width 1) (layer "F.Cu") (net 1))
 (segment (start 165.75 96.25) (end 165.75 98.599022) (width 1) (layer "F.Cu") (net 1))
 (segment (start 165.75 98.599022) (end 161.899022 102.45) (width 1) (layer "F.Cu") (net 1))
 (segment (start 160.6 103) (end 161.15 102.45) (width 1) (layer "F.Cu") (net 1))
 (via (at 155.8 94.75) (size 0.8) (drill 0.4) (layers "F.Cu" "B.Cu") (free) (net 3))
 (via (at 145.8 93) (size 0.8) (drill 0.4) (layers "F.Cu" "B.Cu") (free) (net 3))
 (via (at 159.5 99.8) (size 0.8) (drill 0.4) (layers "F.Cu" "B.Cu") (free) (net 3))
 (via (at 161.75 87.25) (size 0.8) (drill 0.4) (layers "F.Cu" "B.Cu") (free) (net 3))
 (via (at 148.25 81.75) (size 0.8) (drill 0.4) (layers "F.Cu" "B.Cu") (free) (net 3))
 (via (at 167.6 99.8) (size 0.8) (drill 0.4) (layers "F.Cu" "B.Cu") (free) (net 3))
 (via (at 163.15 94.2) (size 0.8) (drill 0.4) (layers "F.Cu" "B.Cu") (free) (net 3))
 (segment (start 156.025 97.9) (end 164 97.9) (width 1) (layer "F.Cu") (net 4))
 (segment (start 161.1 82.45) (end 156.4 82.45) (width 1) (layer "F.Cu") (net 4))
 (segment (start 160.15 97.25) (end 159.5 97.9) (width 1) (layer "F.Cu") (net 4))
 (segment (start 155.899022 85.6) (end 160.15 89.850978) (width 1) (layer "F.Cu") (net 4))
 (segment (start 159.5 97.9) (end 156.025 97.9) (width 1) (layer "F.Cu") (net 4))
 (segment (start 156.4 82.45) (end 153.25 85.6) (width 1) (layer "F.Cu") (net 4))
 (segment (start 160.15 89.850978) (end 160.15 97.25) (width 1) (layer "F.Cu") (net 4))
 (segment (start 164 97.9) (end 164.55 97.35) (width 1) (layer "F.Cu") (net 4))
 (segment (start 153.25 85.6) (end 155.899022 85.6) (width 1) (layer "F.Cu") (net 4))
 (segment (start 153.475978 101.3) (end 156.025 101.3) (width 1) (layer "F.Cu") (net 2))
 (segment (start 149.3 91.35) (end 143.55 85.6) (width 1) (layer "F.Cu") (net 2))
 (segment (start 153.025489 100.849511) (end 153.475978 101.3) (width 1) (layer "F.Cu") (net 2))
 (segment (start 156.75 91.35) (end 153.025489 95.074511) (width 1) (layer "F.Cu") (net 2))
 (segment (start 157.6 91.35) (end 149.3 91.35) (width 1) (layer "F.Cu") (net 2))
 (segment (start 153.025489 95.074511) (end 153.025489 100.849511) (width 1) (layer "F.Cu") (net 2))
 (segment (start 157.6 91.35) (end 156.75 91.35) (width 1) (layer "F.Cu") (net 2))
 (segment (start 167.1 96.6) (end 167.85 97.35) (width 1) (layer "F.Cu") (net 5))
 (segment (start 167.1 93.855) (end 167.1 96.6) (width 1) (layer "F.Cu") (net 5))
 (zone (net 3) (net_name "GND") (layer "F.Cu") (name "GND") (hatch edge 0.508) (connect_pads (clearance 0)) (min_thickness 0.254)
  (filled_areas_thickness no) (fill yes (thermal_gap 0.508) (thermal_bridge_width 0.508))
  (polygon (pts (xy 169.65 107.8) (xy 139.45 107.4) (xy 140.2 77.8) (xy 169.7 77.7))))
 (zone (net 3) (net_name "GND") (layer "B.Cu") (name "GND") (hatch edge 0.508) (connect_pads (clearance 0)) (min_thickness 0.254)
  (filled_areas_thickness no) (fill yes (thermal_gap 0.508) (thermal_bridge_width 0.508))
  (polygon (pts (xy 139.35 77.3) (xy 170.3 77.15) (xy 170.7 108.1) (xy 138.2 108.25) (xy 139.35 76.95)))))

